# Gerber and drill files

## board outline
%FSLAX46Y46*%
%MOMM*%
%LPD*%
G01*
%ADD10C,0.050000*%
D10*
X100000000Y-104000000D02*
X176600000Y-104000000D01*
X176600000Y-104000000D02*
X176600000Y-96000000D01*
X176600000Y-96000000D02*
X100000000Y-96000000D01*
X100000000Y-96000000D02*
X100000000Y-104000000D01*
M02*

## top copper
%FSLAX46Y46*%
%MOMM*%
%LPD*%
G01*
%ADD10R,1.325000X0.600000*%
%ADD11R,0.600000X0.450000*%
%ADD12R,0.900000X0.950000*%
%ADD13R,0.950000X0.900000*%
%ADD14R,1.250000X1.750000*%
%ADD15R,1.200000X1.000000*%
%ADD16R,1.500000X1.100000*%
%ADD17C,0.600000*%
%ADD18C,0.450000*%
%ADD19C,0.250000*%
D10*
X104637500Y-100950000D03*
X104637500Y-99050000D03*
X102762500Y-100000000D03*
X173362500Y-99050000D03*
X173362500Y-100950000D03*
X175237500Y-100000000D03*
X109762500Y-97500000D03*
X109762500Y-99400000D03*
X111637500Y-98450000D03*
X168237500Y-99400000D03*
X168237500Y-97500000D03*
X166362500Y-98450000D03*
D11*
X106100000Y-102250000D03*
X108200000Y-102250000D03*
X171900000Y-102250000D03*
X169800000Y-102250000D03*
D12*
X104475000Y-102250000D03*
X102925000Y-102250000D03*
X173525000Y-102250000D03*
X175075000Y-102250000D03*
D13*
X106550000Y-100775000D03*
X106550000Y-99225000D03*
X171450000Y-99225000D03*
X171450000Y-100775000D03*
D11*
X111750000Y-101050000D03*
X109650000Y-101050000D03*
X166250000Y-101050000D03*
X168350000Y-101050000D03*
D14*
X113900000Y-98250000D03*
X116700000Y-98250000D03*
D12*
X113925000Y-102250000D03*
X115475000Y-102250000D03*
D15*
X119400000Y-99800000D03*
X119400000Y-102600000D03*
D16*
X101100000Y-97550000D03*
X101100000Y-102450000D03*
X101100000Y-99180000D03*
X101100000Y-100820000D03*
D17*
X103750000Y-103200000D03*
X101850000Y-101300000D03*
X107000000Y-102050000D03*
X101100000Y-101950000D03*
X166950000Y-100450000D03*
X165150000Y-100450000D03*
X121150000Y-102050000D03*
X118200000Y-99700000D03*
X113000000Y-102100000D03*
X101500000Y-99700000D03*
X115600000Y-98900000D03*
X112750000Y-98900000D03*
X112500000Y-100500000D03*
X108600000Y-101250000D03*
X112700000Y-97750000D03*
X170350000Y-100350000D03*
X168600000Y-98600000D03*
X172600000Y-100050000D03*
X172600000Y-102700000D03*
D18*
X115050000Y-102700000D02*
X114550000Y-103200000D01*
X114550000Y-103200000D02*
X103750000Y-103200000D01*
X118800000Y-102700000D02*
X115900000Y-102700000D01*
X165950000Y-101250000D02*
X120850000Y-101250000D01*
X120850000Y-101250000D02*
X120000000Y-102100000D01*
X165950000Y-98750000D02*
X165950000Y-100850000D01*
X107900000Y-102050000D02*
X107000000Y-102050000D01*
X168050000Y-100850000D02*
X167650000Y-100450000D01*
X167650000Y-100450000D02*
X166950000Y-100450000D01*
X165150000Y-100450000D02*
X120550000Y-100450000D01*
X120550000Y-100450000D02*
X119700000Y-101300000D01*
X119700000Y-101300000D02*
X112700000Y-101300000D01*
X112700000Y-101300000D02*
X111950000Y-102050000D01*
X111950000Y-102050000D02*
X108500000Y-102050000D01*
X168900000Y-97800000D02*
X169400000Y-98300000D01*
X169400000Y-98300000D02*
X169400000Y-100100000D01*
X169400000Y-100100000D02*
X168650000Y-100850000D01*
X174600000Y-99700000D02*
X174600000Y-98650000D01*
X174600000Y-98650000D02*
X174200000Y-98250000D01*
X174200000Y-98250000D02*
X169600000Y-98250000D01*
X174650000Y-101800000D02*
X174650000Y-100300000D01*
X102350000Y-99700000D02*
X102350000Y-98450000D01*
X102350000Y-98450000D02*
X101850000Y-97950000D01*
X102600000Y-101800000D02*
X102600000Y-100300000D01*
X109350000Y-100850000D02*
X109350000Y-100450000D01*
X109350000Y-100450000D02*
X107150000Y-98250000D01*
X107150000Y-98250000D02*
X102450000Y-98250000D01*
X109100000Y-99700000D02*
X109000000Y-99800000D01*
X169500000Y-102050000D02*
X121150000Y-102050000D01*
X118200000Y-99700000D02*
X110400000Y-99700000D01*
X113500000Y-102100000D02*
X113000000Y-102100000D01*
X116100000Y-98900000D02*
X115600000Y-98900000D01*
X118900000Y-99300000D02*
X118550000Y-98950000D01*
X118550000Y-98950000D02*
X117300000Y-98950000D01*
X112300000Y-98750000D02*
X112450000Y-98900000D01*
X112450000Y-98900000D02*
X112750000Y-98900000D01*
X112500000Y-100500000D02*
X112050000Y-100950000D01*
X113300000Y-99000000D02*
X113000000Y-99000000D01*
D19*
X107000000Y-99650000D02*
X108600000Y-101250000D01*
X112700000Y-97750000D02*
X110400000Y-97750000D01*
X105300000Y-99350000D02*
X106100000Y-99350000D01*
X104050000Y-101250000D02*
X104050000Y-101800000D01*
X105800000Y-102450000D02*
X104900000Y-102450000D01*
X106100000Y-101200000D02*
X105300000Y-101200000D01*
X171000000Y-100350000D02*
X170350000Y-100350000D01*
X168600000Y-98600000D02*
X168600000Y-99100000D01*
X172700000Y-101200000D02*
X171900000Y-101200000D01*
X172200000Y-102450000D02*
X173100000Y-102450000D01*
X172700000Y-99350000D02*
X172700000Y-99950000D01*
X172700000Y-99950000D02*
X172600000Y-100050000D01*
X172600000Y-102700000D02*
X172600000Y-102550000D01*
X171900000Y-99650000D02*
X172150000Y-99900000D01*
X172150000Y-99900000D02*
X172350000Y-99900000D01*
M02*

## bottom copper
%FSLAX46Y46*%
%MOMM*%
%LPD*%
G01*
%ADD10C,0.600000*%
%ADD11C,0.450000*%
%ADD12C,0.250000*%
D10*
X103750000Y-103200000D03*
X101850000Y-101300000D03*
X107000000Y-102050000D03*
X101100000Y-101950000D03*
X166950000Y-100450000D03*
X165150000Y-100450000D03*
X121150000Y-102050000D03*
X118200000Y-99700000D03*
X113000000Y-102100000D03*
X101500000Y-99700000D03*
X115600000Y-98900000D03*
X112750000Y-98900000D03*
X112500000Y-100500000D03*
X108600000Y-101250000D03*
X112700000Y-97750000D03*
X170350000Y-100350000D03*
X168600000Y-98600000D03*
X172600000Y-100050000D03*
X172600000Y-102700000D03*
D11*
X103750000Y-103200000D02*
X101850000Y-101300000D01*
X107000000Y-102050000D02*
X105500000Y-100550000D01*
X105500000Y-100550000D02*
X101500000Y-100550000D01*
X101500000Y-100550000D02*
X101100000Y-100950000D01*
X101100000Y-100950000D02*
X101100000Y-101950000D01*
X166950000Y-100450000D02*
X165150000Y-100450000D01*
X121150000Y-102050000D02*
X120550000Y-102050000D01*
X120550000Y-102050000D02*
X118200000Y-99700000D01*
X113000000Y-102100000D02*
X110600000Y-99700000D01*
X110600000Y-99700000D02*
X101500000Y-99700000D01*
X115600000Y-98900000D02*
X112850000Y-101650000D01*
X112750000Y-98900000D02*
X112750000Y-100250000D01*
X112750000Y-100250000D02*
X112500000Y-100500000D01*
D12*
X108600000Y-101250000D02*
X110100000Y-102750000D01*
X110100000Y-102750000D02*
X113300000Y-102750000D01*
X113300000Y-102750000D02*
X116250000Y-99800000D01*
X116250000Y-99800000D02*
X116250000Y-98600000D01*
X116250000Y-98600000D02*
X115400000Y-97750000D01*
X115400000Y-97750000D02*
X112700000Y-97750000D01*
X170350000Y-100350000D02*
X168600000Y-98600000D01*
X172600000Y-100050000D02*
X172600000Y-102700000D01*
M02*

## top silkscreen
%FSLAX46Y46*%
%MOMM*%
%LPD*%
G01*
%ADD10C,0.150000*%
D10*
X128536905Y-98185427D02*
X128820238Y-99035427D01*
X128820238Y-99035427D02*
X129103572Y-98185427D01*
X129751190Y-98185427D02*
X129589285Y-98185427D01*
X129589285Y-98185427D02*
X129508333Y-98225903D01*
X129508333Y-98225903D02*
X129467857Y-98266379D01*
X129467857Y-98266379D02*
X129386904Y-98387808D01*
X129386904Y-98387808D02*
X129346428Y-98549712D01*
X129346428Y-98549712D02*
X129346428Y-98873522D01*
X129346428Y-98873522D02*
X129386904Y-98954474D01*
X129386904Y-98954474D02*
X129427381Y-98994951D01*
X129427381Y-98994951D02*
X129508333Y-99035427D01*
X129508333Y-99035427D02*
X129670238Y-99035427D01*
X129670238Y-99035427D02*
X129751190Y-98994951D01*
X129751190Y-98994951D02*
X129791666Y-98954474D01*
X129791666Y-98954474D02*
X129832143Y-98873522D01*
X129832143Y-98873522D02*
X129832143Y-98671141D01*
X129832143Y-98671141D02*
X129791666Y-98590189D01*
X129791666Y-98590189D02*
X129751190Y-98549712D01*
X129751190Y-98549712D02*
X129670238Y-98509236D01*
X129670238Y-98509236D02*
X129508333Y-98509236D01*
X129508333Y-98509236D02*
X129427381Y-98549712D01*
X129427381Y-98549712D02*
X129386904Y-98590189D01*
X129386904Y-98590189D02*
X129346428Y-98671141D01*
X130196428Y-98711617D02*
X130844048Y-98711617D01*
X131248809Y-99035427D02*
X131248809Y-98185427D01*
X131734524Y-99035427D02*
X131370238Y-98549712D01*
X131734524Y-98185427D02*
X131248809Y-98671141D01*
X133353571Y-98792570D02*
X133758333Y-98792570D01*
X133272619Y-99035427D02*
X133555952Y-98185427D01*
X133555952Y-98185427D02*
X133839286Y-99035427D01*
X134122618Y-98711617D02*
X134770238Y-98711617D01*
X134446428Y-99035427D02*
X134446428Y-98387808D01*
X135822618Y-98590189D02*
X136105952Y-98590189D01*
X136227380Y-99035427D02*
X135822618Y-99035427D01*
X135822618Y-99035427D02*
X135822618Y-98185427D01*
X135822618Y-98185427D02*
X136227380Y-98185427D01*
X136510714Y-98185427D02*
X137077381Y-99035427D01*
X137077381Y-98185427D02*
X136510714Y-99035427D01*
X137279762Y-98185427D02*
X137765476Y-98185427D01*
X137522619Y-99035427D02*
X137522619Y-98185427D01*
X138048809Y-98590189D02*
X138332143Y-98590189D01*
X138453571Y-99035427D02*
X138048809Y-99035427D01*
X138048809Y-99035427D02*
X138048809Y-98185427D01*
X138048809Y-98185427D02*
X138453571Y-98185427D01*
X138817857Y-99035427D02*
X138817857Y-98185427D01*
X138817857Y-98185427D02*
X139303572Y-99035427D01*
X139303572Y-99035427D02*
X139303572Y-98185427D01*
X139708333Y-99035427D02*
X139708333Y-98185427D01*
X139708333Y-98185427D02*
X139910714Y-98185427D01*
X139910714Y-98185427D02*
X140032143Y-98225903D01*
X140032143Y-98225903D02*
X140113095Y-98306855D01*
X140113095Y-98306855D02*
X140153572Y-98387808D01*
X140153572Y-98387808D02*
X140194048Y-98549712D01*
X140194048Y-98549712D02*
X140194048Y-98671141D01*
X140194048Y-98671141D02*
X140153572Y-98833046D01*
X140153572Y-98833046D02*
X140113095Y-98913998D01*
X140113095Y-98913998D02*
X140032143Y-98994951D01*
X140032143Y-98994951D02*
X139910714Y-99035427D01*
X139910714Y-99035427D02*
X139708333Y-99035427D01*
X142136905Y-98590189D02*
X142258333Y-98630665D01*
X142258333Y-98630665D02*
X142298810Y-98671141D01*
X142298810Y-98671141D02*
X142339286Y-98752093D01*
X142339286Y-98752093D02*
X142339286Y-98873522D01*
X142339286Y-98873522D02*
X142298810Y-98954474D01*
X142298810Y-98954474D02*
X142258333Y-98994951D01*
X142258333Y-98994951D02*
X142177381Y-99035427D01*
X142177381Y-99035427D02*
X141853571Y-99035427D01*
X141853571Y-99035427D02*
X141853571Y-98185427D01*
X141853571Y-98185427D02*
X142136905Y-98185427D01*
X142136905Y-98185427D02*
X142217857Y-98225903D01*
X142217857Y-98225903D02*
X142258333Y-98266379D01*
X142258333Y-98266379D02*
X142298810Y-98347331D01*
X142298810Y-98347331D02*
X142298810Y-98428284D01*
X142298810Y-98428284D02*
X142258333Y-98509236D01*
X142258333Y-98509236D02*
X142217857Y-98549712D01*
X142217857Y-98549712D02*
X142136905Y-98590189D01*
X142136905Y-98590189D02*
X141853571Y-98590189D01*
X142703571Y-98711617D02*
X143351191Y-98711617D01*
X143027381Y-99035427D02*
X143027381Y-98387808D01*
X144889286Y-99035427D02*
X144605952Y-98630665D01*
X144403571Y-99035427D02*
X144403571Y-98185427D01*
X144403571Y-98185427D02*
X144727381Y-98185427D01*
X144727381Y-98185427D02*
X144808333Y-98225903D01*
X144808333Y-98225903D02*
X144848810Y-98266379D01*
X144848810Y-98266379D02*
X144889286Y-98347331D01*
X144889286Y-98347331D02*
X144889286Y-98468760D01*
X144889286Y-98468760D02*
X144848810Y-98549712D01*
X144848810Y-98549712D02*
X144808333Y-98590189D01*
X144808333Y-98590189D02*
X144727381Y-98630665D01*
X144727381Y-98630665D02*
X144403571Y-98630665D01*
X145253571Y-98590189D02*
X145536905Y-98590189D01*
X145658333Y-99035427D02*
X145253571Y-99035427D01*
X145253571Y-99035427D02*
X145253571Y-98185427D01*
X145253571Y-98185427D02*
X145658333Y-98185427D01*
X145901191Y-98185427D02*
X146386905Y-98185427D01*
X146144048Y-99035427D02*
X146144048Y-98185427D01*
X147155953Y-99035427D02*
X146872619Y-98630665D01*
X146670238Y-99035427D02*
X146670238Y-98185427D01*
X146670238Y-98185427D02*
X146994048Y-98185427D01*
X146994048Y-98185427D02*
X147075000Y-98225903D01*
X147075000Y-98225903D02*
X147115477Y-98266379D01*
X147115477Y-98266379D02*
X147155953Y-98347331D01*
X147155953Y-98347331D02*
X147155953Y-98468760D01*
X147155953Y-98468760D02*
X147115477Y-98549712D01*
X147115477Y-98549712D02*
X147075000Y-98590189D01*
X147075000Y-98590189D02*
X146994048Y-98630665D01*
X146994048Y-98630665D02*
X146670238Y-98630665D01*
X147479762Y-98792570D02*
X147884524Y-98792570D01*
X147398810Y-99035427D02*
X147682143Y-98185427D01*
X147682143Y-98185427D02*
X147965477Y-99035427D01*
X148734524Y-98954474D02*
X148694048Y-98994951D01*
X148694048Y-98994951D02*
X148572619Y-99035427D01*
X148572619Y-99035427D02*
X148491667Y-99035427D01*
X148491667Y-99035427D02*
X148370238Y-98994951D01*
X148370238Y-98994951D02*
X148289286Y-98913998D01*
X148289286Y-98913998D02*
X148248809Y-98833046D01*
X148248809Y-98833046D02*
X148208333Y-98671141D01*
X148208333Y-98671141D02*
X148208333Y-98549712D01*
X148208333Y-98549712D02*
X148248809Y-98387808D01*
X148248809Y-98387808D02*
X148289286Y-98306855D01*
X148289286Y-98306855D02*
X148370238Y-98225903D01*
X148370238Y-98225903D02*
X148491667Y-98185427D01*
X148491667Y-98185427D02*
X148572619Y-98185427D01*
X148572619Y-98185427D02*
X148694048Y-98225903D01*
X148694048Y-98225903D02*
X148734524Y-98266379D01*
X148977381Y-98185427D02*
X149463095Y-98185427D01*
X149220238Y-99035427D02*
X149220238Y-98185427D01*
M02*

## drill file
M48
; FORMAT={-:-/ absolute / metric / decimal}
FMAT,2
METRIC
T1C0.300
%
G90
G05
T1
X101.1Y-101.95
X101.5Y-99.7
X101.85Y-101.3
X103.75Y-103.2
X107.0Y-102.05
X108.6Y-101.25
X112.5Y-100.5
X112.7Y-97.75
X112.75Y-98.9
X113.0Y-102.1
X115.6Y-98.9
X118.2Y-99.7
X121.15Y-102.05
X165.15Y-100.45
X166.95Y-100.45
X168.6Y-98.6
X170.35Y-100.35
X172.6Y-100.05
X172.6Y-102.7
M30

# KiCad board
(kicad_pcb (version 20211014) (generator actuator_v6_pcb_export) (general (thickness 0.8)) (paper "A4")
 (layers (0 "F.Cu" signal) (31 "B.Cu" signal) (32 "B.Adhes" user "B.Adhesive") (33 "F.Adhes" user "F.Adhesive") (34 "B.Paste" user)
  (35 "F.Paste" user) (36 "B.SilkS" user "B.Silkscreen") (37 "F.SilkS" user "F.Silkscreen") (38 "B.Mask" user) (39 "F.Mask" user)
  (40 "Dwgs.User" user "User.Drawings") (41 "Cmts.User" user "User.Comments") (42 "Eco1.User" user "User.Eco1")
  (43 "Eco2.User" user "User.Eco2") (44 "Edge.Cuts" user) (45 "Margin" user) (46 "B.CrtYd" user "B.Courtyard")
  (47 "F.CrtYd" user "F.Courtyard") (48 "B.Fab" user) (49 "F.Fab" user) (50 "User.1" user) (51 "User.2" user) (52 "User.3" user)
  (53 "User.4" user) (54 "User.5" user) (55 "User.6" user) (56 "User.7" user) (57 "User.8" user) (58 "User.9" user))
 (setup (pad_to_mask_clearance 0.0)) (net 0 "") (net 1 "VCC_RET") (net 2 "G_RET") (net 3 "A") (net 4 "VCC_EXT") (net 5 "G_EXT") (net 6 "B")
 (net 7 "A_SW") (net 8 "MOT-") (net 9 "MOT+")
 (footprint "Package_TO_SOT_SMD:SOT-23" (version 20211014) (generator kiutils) (layer "F.Cu") (at 103.7 100.0 180)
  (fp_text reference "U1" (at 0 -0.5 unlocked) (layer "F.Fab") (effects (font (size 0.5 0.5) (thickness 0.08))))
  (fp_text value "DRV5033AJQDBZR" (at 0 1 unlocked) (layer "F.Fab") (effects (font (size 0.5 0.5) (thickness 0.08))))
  (pad "1" smd rect (at -0.9375 -0.95 180) (size 1.325 0.6) (layers "F.Cu" "F.Mask" "F.Paste") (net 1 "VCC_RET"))
  (pad "2" smd rect (at -0.9375 0.95 180) (size 1.325 0.6) (layers "F.Cu" "F.Mask" "F.Paste") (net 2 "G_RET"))
  (pad "3" smd rect (at 0.9375 0.0 180) (size 1.325 0.6) (layers "F.Cu" "F.Mask" "F.Paste") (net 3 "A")))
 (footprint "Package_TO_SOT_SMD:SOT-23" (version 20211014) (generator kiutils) (layer "F.Cu") (at 174.3 100.0)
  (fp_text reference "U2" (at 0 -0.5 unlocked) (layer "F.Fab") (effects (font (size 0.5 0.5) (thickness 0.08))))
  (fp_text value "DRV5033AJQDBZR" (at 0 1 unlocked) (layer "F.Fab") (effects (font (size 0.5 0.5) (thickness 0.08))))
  (pad "1" smd rect (at -0.9375 -0.95) (size 1.325 0.6) (layers "F.Cu" "F.Mask" "F.Paste") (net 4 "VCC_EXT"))
  (pad "2" smd rect (at -0.9375 0.95) (size 1.325 0.6) (layers "F.Cu" "F.Mask" "F.Paste") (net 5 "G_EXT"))
  (pad "3" smd rect (at 0.9375 0.0) (size 1.325 0.6) (layers "F.Cu" "F.Mask" "F.Paste") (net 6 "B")))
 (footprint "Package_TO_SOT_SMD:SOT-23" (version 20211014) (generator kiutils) (layer "F.Cu") (at 110.7 98.45)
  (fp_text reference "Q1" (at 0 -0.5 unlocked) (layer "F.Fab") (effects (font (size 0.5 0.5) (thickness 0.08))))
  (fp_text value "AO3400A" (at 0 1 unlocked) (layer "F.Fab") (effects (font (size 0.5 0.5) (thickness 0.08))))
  (pad "1" smd rect (at -0.9375 -0.95) (size 1.325 0.6) (layers "F.Cu" "F.Mask" "F.Paste") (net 2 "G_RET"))
  (pad "2" smd rect (at -0.9375 0.95) (size 1.325 0.6) (layers "F.Cu" "F.Mask" "F.Paste") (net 3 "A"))
  (pad "3" smd rect (at 0.9375 0.0) (size 1.325 0.6) (layers "F.Cu" "F.Mask" "F.Paste") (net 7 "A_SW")))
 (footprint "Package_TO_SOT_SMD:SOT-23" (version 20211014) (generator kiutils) (layer "F.Cu") (at 167.3 98.45 180)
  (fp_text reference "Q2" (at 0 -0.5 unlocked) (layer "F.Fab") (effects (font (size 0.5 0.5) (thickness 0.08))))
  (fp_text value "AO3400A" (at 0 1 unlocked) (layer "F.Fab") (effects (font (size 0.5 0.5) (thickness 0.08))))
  (pad "1" smd rect (at -0.9375 -0.95 180) (size 1.325 0.6) (layers "F.Cu" "F.Mask" "F.Paste") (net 5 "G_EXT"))
  (pad "2" smd rect (at -0.9375 0.95 180) (size 1.325 0.6) (layers "F.Cu" "F.Mask" "F.Paste") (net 6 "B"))
  (pad "3" smd rect (at 0.9375 0.0 180) (size 1.325 0.6) (layers "F.Cu" "F.Mask" "F.Paste") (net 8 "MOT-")))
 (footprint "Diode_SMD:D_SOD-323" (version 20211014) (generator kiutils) (layer "F.Cu") (at 107.15 102.25)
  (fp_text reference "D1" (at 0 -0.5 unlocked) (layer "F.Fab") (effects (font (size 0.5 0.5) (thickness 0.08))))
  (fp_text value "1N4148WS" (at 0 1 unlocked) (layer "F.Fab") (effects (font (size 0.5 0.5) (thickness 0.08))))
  (pad "1" smd rect (at -1.05 0.0) (size 0.6 0.45) (layers "F.Cu" "F.Mask" "F.Paste") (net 1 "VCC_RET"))
  (pad "2" smd rect (at 1.05 0.0) (size 0.6 0.45) (layers "F.Cu" "F.Mask" "F.Paste") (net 6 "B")))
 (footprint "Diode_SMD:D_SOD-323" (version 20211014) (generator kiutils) (layer "F.Cu") (at 170.85 102.25 180)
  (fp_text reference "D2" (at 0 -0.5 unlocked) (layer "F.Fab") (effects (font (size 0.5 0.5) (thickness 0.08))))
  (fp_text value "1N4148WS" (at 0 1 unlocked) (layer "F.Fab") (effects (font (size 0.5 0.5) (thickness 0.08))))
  (pad "1" smd rect (at -1.05 0.0 180) (size 0.6 0.45) (layers "F.Cu" "F.Mask" "F.Paste") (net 4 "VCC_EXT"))
  (pad "2" smd rect (at 1.05 0.0 180) (size 0.6 0.45) (layers "F.Cu" "F.Mask" "F.Paste") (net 3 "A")))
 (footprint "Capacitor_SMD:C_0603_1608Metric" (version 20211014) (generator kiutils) (layer "F.Cu") (at 103.7 102.25 180)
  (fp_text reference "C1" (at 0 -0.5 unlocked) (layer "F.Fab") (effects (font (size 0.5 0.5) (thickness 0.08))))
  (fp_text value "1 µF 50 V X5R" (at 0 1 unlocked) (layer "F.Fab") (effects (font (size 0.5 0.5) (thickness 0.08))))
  (pad "1" smd rect (at -0.775 0.0 180) (size 0.9 0.95) (layers "F.Cu" "F.Mask" "F.Paste") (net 1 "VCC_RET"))
  (pad "2" smd rect (at 0.775 0.0 180) (size 0.9 0.95) (layers "F.Cu" "F.Mask" "F.Paste") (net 3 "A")))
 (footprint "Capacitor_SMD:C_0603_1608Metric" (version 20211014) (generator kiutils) (layer "F.Cu") (at 174.3 102.25)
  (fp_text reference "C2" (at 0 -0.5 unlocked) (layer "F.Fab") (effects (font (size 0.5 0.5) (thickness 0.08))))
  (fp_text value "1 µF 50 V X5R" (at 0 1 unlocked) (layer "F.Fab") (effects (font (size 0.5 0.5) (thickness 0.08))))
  (pad "1" smd rect (at -0.775 0.0) (size 0.9 0.95) (layers "F.Cu" "F.Mask" "F.Paste") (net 4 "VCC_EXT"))
  (pad "2" smd rect (at 0.775 0.0) (size 0.9 0.95) (layers "F.Cu" "F.Mask" "F.Paste") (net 6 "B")))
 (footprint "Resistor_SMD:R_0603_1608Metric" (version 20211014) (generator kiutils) (layer "F.Cu") (at 106.55 100.0 90)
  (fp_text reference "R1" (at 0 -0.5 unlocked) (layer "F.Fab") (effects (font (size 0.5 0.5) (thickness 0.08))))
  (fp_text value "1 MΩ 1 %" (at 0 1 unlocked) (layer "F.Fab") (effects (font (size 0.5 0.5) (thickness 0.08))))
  (pad "1" smd rect (at -0.775 0.0 90) (size 0.9 0.95) (layers "F.Cu" "F.Mask" "F.Paste") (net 1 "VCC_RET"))
  (pad "2" smd rect (at 0.775 0.0 90) (size 0.9 0.95) (layers "F.Cu" "F.Mask" "F.Paste") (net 2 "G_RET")))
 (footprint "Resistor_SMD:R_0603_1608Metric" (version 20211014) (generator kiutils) (layer "F.Cu") (at 171.45 100.0 270)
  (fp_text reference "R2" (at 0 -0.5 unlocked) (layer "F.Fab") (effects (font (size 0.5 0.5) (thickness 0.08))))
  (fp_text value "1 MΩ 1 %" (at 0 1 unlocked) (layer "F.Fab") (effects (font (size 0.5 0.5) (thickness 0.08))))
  (pad "1" smd rect (at -0.775 0.0 270) (size 0.9 0.95) (layers "F.Cu" "F.Mask" "F.Paste") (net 4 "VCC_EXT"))
  (pad "2" smd rect (at 0.775 0.0 270) (size 0.9 0.95) (layers "F.Cu" "F.Mask" "F.Paste") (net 5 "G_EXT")))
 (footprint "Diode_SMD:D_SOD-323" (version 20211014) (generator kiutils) (layer "F.Cu") (at 110.7 101.05 180)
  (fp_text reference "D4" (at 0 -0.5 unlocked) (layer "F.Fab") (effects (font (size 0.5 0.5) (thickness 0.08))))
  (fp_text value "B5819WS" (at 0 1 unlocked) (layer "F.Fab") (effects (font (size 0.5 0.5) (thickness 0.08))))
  (pad "1" smd rect (at -1.05 0.0 180) (size 0.6 0.45) (layers "F.Cu" "F.Mask" "F.Paste") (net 7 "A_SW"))
  (pad "2" smd rect (at 1.05 0.0 180) (size 0.6 0.45) (layers "F.Cu" "F.Mask" "F.Paste") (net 3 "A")))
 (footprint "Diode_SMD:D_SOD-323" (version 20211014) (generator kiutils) (layer "F.Cu") (at 167.3 101.05)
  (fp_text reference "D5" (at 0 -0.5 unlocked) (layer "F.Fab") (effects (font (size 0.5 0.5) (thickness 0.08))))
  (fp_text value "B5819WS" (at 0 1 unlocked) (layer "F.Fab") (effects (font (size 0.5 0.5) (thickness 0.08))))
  (pad "1" smd rect (at -1.05 0.0) (size 0.6 0.45) (layers "F.Cu" "F.Mask" "F.Paste") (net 8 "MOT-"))
  (pad "2" smd rect (at 1.05 0.0) (size 0.6 0.45) (layers "F.Cu" "F.Mask" "F.Paste") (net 6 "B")))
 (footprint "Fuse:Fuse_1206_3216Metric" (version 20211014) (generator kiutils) (layer "F.Cu") (at 115.3 98.25)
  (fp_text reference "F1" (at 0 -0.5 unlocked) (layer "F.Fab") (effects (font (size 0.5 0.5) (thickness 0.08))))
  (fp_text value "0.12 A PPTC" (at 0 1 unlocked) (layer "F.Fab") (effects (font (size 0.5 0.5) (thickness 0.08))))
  (pad "1" smd rect (at -1.4 0.0) (size 1.25 1.75) (layers "F.Cu" "F.Mask" "F.Paste") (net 7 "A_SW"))
  (pad "2" smd rect (at 1.4 0.0) (size 1.25 1.75) (layers "F.Cu" "F.Mask" "F.Paste") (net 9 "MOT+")))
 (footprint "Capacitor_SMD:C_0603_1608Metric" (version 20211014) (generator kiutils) (layer "F.Cu") (at 114.7 102.25)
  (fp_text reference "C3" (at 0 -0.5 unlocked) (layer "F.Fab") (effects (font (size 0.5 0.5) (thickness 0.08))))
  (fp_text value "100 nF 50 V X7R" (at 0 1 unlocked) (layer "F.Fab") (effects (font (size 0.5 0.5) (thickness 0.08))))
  (pad "1" smd rect (at -0.775 0.0) (size 0.9 0.95) (layers "F.Cu" "F.Mask" "F.Paste") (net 9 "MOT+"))
  (pad "2" smd rect (at 0.775 0.0) (size 0.9 0.95) (layers "F.Cu" "F.Mask" "F.Paste") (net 8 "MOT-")))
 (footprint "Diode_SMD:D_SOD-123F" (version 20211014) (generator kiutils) (layer "F.Cu") (at 119.4 101.2 270)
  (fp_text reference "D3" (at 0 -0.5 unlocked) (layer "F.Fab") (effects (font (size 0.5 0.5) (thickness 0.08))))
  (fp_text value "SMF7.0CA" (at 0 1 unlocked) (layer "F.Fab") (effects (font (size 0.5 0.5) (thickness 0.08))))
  (pad "1" smd rect (at -1.4 0.0 270) (size 1.0 1.2) (layers "F.Cu" "F.Mask" "F.Paste") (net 9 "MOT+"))
  (pad "2" smd rect (at 1.4 0.0 270) (size 1.0 1.2) (layers "F.Cu" "F.Mask" "F.Paste") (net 8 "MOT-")))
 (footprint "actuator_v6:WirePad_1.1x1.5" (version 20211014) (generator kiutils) (layer "F.Cu") (at 101.1 97.55)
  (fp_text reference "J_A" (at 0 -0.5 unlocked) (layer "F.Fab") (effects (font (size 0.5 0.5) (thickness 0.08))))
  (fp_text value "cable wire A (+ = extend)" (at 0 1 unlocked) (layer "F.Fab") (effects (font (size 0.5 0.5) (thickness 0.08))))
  (pad "1" smd rect (at 0.0 0.0) (size 1.5 1.1) (layers "F.Cu" "F.Mask") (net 3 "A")))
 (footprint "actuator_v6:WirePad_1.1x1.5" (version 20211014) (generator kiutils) (layer "F.Cu") (at 101.1 102.45)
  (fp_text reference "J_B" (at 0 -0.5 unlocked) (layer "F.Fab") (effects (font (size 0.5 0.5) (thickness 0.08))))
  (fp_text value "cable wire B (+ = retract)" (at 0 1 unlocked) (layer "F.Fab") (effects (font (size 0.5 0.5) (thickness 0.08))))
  (pad "1" smd rect (at 0.0 0.0) (size 1.5 1.1) (layers "F.Cu" "F.Mask") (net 6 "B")))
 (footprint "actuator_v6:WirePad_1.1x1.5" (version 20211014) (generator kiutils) (layer "F.Cu") (at 101.1 99.18)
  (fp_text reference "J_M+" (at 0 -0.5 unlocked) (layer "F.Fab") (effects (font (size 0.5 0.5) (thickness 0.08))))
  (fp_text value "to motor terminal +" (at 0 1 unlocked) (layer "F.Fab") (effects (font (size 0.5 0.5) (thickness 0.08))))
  (pad "1" smd rect (at 0.0 0.0) (size 1.5 1.1) (layers "F.Cu" "F.Mask") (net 9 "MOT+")))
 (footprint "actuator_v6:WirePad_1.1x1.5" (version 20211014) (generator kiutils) (layer "F.Cu") (at 101.1 100.82)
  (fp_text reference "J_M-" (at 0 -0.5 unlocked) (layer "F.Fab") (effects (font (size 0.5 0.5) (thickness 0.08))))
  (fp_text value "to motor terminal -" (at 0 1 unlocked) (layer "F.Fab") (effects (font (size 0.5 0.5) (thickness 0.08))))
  (pad "1" smd rect (at 0.0 0.0) (size 1.5 1.1) (layers "F.Cu" "F.Mask") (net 8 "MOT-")))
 (gr_line (start 100.0 104.0) (end 176.6 104.0) (layer "Edge.Cuts") (width 0.05))
 (gr_line (start 176.6 104.0) (end 176.6 96.0) (layer "Edge.Cuts") (width 0.05))
 (gr_line (start 176.6 96.0) (end 100.0 96.0) (layer "Edge.Cuts") (width 0.05))
 (gr_line (start 100.0 96.0) (end 100.0 104.0) (layer "Edge.Cuts") (width 0.05))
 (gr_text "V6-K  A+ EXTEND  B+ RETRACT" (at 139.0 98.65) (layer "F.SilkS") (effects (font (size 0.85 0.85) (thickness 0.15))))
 (segment (start 115.05 102.7) (end 114.55 103.2) (width 0.45) (layer "F.Cu") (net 8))
 (segment (start 114.55 103.2) (end 103.75 103.2) (width 0.45) (layer "F.Cu") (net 8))
 (segment (start 103.75 103.2) (end 101.85 101.3) (width 0.45) (layer "B.Cu") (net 8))
 (segment (start 118.8 102.7) (end 115.9 102.7) (width 0.45) (layer "F.Cu") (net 8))
 (segment (start 165.95 101.25) (end 120.85 101.25) (width 0.45) (layer "F.Cu") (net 8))
 (segment (start 120.85 101.25) (end 120.0 102.1) (width 0.45) (layer "F.Cu") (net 8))
 (segment (start 165.95 98.75) (end 165.95 100.85) (width 0.45) (layer "F.Cu") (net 8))
 (segment (start 107.9 102.05) (end 107.0 102.05) (width 0.45) (layer "F.Cu") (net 6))
 (segment (start 107.0 102.05) (end 105.5 100.55) (width 0.45) (layer "B.Cu") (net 6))
 (segment (start 105.5 100.55) (end 101.5 100.55) (width 0.45) (layer "B.Cu") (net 6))
 (segment (start 101.5 100.55) (end 101.1 100.95) (width 0.45) (layer "B.Cu") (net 6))
 (segment (start 101.1 100.95) (end 101.1 101.95) (width 0.45) (layer "B.Cu") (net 6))
 (segment (start 168.05 100.85) (end 167.65 100.45) (width 0.45) (layer "F.Cu") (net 6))
 (segment (start 167.65 100.45) (end 166.95 100.45) (width 0.45) (layer "F.Cu") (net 6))
 (segment (start 166.95 100.45) (end 165.15 100.45) (width 0.45) (layer "B.Cu") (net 6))
 (segment (start 165.15 100.45) (end 120.55 100.45) (width 0.45) (layer "F.Cu") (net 6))
 (segment (start 120.55 100.45) (end 119.7 101.3) (width 0.45) (layer "F.Cu") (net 6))
 (segment (start 119.7 101.3) (end 112.7 101.3) (width 0.45) (layer "F.Cu") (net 6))
 (segment (start 112.7 101.3) (end 111.95 102.05) (width 0.45) (layer "F.Cu") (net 6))
 (segment (start 111.95 102.05) (end 108.5 102.05) (width 0.45) (layer "F.Cu") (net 6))
 (segment (start 168.9 97.8) (end 169.4 98.3) (width 0.45) (layer "F.Cu") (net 6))
 (segment (start 169.4 98.3) (end 169.4 100.1) (width 0.45) (layer "F.Cu") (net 6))
 (segment (start 169.4 100.1) (end 168.65 100.85) (width 0.45) (layer "F.Cu") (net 6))
 (segment (start 174.6 99.7) (end 174.6 98.65) (width 0.45) (layer "F.Cu") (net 6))
 (segment (start 174.6 98.65) (end 174.2 98.25) (width 0.45) (layer "F.Cu") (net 6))
 (segment (start 174.2 98.25) (end 169.6 98.25) (width 0.45) (layer "F.Cu") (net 6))
 (segment (start 174.65 101.8) (end 174.65 100.3) (width 0.45) (layer "F.Cu") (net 6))
 (segment (start 102.35 99.7) (end 102.35 98.45) (width 0.45) (layer "F.Cu") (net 3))
 (segment (start 102.35 98.45) (end 101.85 97.95) (width 0.45) (layer "F.Cu") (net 3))
 (segment (start 102.6 101.8) (end 102.6 100.3) (width 0.45) (layer "F.Cu") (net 3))
 (segment (start 109.35 100.85) (end 109.35 100.45) (width 0.45) (layer "F.Cu") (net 3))
 (segment (start 109.35 100.45) (end 107.15 98.25) (width 0.45) (layer "F.Cu") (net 3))
 (segment (start 107.15 98.25) (end 102.45 98.25) (width 0.45) (layer "F.Cu") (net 3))
 (segment (start 109.1 99.7) (end 109.0 99.8) (width 0.45) (layer "F.Cu") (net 3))
 (segment (start 169.5 102.05) (end 121.15 102.05) (width 0.45) (layer "F.Cu") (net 3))
 (segment (start 121.15 102.05) (end 120.55 102.05) (width 0.45) (layer "B.Cu") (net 3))
 (segment (start 120.55 102.05) (end 118.2 99.7) (width 0.45) (layer "B.Cu") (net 3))
 (segment (start 118.2 99.7) (end 110.4 99.7) (width 0.45) (layer "F.Cu") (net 3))
 (segment (start 113.5 102.1) (end 113.0 102.1) (width 0.45) (layer "F.Cu") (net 9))
 (segment (start 113.0 102.1) (end 110.6 99.7) (width 0.45) (layer "B.Cu") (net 9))
 (segment (start 110.6 99.7) (end 101.5 99.7) (width 0.45) (layer "B.Cu") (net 9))
 (segment (start 116.1 98.9) (end 115.6 98.9) (width 0.45) (layer "F.Cu") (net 9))
 (segment (start 115.6 98.9) (end 112.85 101.65) (width 0.45) (layer "B.Cu") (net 9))
 (segment (start 118.9 99.3) (end 118.55 98.95) (width 0.45) (layer "F.Cu") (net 9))
 (segment (start 118.55 98.95) (end 117.3 98.95) (width 0.45) (layer "F.Cu") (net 9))
 (segment (start 112.3 98.75) (end 112.45 98.9) (width 0.45) (layer "F.Cu") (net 7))
 (segment (start 112.45 98.9) (end 112.75 98.9) (width 0.45) (layer "F.Cu") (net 7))
 (segment (start 112.75 98.9) (end 112.75 100.25) (width 0.45) (layer "B.Cu") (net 7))
 (segment (start 112.75 100.25) (end 112.5 100.5) (width 0.45) (layer "B.Cu") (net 7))
 (segment (start 112.5 100.5) (end 112.05 100.95) (width 0.45) (layer "F.Cu") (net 7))
 (segment (start 113.3 99.0) (end 113.0 99.0) (width 0.45) (layer "F.Cu") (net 7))
 (segment (start 107.0 99.65) (end 108.6 101.25) (width 0.25) (layer "F.Cu") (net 2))
 (segment (start 108.6 101.25) (end 110.1 102.75) (width 0.25) (layer "B.Cu") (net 2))
 (segment (start 110.1 102.75) (end 113.3 102.75) (width 0.25) (layer "B.Cu") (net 2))
 (segment (start 113.3 102.75) (end 116.25 99.8) (width 0.25) (layer "B.Cu") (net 2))
 (segment (start 116.25 99.8) (end 116.25 98.6) (width 0.25) (layer "B.Cu") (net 2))
 (segment (start 116.25 98.6) (end 115.4 97.75) (width 0.25) (layer "B.Cu") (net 2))
 (segment (start 115.4 97.75) (end 112.7 97.75) (width 0.25) (layer "B.Cu") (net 2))
 (segment (start 112.7 97.75) (end 110.4 97.75) (width 0.25) (layer "F.Cu") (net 2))
 (segment (start 105.3 99.35) (end 106.1 99.35) (width 0.25) (layer "F.Cu") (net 2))
 (segment (start 104.05 101.25) (end 104.05 101.8) (width 0.25) (layer "F.Cu") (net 1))
 (segment (start 105.8 102.45) (end 104.9 102.45) (width 0.25) (layer "F.Cu") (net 1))
 (segment (start 106.1 101.2) (end 105.3 101.2) (width 0.25) (layer "F.Cu") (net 1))
 (segment (start 171.0 100.35) (end 170.35 100.35) (width 0.25) (layer "F.Cu") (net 5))
 (segment (start 170.35 100.35) (end 168.6 98.6) (width 0.25) (layer "B.Cu") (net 5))
 (segment (start 168.6 98.6) (end 168.6 99.1) (width 0.25) (layer "F.Cu") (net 5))
 (segment (start 172.7 101.2) (end 171.9 101.2) (width 0.25) (layer "F.Cu") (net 5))
 (segment (start 172.2 102.45) (end 173.1 102.45) (width 0.25) (layer "F.Cu") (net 4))
 (segment (start 172.7 99.35) (end 172.7 99.95) (width 0.25) (layer "F.Cu") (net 4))
 (segment (start 172.7 99.95) (end 172.6 100.05) (width 0.25) (layer "F.Cu") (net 4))
 (segment (start 172.6 100.05) (end 172.6 102.7) (width 0.25) (layer "B.Cu") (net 4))
 (segment (start 172.6 102.7) (end 172.6 102.55) (width 0.25) (layer "F.Cu") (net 4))
 (segment (start 171.9 99.65) (end 172.15 99.9) (width 0.25) (layer "F.Cu") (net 4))
 (segment (start 172.15 99.9) (end 172.35 99.9) (width 0.25) (layer "F.Cu") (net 4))
 (via (at 103.75 103.2) (size 0.6) (drill 0.3) (layers "F.Cu" "B.Cu") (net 8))
 (via (at 101.85 101.3) (size 0.6) (drill 0.3) (layers "F.Cu" "B.Cu") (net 8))
 (via (at 107.0 102.05) (size 0.6) (drill 0.3) (layers "F.Cu" "B.Cu") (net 6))
 (via (at 101.1 101.95) (size 0.6) (drill 0.3) (layers "F.Cu" "B.Cu") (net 6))
 (via (at 166.95 100.45) (size 0.6) (drill 0.3) (layers "F.Cu" "B.Cu") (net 6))
 (via (at 165.15 100.45) (size 0.6) (drill 0.3) (layers "F.Cu" "B.Cu") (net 6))
 (via (at 121.15 102.05) (size 0.6) (drill 0.3) (layers "F.Cu" "B.Cu") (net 3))
 (via (at 118.2 99.7) (size 0.6) (drill 0.3) (layers "F.Cu" "B.Cu") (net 3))
 (via (at 113.0 102.1) (size 0.6) (drill 0.3) (layers "F.Cu" "B.Cu") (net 9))
 (via (at 101.5 99.7) (size 0.6) (drill 0.3) (layers "F.Cu" "B.Cu") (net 9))
 (via (at 115.6 98.9) (size 0.6) (drill 0.3) (layers "F.Cu" "B.Cu") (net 9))
 (via (at 112.75 98.9) (size 0.6) (drill 0.3) (layers "F.Cu" "B.Cu") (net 7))
 (via (at 112.5 100.5) (size 0.6) (drill 0.3) (layers "F.Cu" "B.Cu") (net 7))
 (via (at 108.6 101.25) (size 0.6) (drill 0.3) (layers "F.Cu" "B.Cu") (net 2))
 (via (at 112.7 97.75) (size 0.6) (drill 0.3) (layers "F.Cu" "B.Cu") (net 2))
 (via (at 170.35 100.35) (size 0.6) (drill 0.3) (layers "F.Cu" "B.Cu") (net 5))
 (via (at 168.6 98.6) (size 0.6) (drill 0.3) (layers "F.Cu" "B.Cu") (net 5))
 (via (at 172.6 100.05) (size 0.6) (drill 0.3) (layers "F.Cu" "B.Cu") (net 4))
 (via (at 172.6 102.7) (size 0.6) (drill 0.3) (layers "F.Cu" "B.Cu") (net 4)))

